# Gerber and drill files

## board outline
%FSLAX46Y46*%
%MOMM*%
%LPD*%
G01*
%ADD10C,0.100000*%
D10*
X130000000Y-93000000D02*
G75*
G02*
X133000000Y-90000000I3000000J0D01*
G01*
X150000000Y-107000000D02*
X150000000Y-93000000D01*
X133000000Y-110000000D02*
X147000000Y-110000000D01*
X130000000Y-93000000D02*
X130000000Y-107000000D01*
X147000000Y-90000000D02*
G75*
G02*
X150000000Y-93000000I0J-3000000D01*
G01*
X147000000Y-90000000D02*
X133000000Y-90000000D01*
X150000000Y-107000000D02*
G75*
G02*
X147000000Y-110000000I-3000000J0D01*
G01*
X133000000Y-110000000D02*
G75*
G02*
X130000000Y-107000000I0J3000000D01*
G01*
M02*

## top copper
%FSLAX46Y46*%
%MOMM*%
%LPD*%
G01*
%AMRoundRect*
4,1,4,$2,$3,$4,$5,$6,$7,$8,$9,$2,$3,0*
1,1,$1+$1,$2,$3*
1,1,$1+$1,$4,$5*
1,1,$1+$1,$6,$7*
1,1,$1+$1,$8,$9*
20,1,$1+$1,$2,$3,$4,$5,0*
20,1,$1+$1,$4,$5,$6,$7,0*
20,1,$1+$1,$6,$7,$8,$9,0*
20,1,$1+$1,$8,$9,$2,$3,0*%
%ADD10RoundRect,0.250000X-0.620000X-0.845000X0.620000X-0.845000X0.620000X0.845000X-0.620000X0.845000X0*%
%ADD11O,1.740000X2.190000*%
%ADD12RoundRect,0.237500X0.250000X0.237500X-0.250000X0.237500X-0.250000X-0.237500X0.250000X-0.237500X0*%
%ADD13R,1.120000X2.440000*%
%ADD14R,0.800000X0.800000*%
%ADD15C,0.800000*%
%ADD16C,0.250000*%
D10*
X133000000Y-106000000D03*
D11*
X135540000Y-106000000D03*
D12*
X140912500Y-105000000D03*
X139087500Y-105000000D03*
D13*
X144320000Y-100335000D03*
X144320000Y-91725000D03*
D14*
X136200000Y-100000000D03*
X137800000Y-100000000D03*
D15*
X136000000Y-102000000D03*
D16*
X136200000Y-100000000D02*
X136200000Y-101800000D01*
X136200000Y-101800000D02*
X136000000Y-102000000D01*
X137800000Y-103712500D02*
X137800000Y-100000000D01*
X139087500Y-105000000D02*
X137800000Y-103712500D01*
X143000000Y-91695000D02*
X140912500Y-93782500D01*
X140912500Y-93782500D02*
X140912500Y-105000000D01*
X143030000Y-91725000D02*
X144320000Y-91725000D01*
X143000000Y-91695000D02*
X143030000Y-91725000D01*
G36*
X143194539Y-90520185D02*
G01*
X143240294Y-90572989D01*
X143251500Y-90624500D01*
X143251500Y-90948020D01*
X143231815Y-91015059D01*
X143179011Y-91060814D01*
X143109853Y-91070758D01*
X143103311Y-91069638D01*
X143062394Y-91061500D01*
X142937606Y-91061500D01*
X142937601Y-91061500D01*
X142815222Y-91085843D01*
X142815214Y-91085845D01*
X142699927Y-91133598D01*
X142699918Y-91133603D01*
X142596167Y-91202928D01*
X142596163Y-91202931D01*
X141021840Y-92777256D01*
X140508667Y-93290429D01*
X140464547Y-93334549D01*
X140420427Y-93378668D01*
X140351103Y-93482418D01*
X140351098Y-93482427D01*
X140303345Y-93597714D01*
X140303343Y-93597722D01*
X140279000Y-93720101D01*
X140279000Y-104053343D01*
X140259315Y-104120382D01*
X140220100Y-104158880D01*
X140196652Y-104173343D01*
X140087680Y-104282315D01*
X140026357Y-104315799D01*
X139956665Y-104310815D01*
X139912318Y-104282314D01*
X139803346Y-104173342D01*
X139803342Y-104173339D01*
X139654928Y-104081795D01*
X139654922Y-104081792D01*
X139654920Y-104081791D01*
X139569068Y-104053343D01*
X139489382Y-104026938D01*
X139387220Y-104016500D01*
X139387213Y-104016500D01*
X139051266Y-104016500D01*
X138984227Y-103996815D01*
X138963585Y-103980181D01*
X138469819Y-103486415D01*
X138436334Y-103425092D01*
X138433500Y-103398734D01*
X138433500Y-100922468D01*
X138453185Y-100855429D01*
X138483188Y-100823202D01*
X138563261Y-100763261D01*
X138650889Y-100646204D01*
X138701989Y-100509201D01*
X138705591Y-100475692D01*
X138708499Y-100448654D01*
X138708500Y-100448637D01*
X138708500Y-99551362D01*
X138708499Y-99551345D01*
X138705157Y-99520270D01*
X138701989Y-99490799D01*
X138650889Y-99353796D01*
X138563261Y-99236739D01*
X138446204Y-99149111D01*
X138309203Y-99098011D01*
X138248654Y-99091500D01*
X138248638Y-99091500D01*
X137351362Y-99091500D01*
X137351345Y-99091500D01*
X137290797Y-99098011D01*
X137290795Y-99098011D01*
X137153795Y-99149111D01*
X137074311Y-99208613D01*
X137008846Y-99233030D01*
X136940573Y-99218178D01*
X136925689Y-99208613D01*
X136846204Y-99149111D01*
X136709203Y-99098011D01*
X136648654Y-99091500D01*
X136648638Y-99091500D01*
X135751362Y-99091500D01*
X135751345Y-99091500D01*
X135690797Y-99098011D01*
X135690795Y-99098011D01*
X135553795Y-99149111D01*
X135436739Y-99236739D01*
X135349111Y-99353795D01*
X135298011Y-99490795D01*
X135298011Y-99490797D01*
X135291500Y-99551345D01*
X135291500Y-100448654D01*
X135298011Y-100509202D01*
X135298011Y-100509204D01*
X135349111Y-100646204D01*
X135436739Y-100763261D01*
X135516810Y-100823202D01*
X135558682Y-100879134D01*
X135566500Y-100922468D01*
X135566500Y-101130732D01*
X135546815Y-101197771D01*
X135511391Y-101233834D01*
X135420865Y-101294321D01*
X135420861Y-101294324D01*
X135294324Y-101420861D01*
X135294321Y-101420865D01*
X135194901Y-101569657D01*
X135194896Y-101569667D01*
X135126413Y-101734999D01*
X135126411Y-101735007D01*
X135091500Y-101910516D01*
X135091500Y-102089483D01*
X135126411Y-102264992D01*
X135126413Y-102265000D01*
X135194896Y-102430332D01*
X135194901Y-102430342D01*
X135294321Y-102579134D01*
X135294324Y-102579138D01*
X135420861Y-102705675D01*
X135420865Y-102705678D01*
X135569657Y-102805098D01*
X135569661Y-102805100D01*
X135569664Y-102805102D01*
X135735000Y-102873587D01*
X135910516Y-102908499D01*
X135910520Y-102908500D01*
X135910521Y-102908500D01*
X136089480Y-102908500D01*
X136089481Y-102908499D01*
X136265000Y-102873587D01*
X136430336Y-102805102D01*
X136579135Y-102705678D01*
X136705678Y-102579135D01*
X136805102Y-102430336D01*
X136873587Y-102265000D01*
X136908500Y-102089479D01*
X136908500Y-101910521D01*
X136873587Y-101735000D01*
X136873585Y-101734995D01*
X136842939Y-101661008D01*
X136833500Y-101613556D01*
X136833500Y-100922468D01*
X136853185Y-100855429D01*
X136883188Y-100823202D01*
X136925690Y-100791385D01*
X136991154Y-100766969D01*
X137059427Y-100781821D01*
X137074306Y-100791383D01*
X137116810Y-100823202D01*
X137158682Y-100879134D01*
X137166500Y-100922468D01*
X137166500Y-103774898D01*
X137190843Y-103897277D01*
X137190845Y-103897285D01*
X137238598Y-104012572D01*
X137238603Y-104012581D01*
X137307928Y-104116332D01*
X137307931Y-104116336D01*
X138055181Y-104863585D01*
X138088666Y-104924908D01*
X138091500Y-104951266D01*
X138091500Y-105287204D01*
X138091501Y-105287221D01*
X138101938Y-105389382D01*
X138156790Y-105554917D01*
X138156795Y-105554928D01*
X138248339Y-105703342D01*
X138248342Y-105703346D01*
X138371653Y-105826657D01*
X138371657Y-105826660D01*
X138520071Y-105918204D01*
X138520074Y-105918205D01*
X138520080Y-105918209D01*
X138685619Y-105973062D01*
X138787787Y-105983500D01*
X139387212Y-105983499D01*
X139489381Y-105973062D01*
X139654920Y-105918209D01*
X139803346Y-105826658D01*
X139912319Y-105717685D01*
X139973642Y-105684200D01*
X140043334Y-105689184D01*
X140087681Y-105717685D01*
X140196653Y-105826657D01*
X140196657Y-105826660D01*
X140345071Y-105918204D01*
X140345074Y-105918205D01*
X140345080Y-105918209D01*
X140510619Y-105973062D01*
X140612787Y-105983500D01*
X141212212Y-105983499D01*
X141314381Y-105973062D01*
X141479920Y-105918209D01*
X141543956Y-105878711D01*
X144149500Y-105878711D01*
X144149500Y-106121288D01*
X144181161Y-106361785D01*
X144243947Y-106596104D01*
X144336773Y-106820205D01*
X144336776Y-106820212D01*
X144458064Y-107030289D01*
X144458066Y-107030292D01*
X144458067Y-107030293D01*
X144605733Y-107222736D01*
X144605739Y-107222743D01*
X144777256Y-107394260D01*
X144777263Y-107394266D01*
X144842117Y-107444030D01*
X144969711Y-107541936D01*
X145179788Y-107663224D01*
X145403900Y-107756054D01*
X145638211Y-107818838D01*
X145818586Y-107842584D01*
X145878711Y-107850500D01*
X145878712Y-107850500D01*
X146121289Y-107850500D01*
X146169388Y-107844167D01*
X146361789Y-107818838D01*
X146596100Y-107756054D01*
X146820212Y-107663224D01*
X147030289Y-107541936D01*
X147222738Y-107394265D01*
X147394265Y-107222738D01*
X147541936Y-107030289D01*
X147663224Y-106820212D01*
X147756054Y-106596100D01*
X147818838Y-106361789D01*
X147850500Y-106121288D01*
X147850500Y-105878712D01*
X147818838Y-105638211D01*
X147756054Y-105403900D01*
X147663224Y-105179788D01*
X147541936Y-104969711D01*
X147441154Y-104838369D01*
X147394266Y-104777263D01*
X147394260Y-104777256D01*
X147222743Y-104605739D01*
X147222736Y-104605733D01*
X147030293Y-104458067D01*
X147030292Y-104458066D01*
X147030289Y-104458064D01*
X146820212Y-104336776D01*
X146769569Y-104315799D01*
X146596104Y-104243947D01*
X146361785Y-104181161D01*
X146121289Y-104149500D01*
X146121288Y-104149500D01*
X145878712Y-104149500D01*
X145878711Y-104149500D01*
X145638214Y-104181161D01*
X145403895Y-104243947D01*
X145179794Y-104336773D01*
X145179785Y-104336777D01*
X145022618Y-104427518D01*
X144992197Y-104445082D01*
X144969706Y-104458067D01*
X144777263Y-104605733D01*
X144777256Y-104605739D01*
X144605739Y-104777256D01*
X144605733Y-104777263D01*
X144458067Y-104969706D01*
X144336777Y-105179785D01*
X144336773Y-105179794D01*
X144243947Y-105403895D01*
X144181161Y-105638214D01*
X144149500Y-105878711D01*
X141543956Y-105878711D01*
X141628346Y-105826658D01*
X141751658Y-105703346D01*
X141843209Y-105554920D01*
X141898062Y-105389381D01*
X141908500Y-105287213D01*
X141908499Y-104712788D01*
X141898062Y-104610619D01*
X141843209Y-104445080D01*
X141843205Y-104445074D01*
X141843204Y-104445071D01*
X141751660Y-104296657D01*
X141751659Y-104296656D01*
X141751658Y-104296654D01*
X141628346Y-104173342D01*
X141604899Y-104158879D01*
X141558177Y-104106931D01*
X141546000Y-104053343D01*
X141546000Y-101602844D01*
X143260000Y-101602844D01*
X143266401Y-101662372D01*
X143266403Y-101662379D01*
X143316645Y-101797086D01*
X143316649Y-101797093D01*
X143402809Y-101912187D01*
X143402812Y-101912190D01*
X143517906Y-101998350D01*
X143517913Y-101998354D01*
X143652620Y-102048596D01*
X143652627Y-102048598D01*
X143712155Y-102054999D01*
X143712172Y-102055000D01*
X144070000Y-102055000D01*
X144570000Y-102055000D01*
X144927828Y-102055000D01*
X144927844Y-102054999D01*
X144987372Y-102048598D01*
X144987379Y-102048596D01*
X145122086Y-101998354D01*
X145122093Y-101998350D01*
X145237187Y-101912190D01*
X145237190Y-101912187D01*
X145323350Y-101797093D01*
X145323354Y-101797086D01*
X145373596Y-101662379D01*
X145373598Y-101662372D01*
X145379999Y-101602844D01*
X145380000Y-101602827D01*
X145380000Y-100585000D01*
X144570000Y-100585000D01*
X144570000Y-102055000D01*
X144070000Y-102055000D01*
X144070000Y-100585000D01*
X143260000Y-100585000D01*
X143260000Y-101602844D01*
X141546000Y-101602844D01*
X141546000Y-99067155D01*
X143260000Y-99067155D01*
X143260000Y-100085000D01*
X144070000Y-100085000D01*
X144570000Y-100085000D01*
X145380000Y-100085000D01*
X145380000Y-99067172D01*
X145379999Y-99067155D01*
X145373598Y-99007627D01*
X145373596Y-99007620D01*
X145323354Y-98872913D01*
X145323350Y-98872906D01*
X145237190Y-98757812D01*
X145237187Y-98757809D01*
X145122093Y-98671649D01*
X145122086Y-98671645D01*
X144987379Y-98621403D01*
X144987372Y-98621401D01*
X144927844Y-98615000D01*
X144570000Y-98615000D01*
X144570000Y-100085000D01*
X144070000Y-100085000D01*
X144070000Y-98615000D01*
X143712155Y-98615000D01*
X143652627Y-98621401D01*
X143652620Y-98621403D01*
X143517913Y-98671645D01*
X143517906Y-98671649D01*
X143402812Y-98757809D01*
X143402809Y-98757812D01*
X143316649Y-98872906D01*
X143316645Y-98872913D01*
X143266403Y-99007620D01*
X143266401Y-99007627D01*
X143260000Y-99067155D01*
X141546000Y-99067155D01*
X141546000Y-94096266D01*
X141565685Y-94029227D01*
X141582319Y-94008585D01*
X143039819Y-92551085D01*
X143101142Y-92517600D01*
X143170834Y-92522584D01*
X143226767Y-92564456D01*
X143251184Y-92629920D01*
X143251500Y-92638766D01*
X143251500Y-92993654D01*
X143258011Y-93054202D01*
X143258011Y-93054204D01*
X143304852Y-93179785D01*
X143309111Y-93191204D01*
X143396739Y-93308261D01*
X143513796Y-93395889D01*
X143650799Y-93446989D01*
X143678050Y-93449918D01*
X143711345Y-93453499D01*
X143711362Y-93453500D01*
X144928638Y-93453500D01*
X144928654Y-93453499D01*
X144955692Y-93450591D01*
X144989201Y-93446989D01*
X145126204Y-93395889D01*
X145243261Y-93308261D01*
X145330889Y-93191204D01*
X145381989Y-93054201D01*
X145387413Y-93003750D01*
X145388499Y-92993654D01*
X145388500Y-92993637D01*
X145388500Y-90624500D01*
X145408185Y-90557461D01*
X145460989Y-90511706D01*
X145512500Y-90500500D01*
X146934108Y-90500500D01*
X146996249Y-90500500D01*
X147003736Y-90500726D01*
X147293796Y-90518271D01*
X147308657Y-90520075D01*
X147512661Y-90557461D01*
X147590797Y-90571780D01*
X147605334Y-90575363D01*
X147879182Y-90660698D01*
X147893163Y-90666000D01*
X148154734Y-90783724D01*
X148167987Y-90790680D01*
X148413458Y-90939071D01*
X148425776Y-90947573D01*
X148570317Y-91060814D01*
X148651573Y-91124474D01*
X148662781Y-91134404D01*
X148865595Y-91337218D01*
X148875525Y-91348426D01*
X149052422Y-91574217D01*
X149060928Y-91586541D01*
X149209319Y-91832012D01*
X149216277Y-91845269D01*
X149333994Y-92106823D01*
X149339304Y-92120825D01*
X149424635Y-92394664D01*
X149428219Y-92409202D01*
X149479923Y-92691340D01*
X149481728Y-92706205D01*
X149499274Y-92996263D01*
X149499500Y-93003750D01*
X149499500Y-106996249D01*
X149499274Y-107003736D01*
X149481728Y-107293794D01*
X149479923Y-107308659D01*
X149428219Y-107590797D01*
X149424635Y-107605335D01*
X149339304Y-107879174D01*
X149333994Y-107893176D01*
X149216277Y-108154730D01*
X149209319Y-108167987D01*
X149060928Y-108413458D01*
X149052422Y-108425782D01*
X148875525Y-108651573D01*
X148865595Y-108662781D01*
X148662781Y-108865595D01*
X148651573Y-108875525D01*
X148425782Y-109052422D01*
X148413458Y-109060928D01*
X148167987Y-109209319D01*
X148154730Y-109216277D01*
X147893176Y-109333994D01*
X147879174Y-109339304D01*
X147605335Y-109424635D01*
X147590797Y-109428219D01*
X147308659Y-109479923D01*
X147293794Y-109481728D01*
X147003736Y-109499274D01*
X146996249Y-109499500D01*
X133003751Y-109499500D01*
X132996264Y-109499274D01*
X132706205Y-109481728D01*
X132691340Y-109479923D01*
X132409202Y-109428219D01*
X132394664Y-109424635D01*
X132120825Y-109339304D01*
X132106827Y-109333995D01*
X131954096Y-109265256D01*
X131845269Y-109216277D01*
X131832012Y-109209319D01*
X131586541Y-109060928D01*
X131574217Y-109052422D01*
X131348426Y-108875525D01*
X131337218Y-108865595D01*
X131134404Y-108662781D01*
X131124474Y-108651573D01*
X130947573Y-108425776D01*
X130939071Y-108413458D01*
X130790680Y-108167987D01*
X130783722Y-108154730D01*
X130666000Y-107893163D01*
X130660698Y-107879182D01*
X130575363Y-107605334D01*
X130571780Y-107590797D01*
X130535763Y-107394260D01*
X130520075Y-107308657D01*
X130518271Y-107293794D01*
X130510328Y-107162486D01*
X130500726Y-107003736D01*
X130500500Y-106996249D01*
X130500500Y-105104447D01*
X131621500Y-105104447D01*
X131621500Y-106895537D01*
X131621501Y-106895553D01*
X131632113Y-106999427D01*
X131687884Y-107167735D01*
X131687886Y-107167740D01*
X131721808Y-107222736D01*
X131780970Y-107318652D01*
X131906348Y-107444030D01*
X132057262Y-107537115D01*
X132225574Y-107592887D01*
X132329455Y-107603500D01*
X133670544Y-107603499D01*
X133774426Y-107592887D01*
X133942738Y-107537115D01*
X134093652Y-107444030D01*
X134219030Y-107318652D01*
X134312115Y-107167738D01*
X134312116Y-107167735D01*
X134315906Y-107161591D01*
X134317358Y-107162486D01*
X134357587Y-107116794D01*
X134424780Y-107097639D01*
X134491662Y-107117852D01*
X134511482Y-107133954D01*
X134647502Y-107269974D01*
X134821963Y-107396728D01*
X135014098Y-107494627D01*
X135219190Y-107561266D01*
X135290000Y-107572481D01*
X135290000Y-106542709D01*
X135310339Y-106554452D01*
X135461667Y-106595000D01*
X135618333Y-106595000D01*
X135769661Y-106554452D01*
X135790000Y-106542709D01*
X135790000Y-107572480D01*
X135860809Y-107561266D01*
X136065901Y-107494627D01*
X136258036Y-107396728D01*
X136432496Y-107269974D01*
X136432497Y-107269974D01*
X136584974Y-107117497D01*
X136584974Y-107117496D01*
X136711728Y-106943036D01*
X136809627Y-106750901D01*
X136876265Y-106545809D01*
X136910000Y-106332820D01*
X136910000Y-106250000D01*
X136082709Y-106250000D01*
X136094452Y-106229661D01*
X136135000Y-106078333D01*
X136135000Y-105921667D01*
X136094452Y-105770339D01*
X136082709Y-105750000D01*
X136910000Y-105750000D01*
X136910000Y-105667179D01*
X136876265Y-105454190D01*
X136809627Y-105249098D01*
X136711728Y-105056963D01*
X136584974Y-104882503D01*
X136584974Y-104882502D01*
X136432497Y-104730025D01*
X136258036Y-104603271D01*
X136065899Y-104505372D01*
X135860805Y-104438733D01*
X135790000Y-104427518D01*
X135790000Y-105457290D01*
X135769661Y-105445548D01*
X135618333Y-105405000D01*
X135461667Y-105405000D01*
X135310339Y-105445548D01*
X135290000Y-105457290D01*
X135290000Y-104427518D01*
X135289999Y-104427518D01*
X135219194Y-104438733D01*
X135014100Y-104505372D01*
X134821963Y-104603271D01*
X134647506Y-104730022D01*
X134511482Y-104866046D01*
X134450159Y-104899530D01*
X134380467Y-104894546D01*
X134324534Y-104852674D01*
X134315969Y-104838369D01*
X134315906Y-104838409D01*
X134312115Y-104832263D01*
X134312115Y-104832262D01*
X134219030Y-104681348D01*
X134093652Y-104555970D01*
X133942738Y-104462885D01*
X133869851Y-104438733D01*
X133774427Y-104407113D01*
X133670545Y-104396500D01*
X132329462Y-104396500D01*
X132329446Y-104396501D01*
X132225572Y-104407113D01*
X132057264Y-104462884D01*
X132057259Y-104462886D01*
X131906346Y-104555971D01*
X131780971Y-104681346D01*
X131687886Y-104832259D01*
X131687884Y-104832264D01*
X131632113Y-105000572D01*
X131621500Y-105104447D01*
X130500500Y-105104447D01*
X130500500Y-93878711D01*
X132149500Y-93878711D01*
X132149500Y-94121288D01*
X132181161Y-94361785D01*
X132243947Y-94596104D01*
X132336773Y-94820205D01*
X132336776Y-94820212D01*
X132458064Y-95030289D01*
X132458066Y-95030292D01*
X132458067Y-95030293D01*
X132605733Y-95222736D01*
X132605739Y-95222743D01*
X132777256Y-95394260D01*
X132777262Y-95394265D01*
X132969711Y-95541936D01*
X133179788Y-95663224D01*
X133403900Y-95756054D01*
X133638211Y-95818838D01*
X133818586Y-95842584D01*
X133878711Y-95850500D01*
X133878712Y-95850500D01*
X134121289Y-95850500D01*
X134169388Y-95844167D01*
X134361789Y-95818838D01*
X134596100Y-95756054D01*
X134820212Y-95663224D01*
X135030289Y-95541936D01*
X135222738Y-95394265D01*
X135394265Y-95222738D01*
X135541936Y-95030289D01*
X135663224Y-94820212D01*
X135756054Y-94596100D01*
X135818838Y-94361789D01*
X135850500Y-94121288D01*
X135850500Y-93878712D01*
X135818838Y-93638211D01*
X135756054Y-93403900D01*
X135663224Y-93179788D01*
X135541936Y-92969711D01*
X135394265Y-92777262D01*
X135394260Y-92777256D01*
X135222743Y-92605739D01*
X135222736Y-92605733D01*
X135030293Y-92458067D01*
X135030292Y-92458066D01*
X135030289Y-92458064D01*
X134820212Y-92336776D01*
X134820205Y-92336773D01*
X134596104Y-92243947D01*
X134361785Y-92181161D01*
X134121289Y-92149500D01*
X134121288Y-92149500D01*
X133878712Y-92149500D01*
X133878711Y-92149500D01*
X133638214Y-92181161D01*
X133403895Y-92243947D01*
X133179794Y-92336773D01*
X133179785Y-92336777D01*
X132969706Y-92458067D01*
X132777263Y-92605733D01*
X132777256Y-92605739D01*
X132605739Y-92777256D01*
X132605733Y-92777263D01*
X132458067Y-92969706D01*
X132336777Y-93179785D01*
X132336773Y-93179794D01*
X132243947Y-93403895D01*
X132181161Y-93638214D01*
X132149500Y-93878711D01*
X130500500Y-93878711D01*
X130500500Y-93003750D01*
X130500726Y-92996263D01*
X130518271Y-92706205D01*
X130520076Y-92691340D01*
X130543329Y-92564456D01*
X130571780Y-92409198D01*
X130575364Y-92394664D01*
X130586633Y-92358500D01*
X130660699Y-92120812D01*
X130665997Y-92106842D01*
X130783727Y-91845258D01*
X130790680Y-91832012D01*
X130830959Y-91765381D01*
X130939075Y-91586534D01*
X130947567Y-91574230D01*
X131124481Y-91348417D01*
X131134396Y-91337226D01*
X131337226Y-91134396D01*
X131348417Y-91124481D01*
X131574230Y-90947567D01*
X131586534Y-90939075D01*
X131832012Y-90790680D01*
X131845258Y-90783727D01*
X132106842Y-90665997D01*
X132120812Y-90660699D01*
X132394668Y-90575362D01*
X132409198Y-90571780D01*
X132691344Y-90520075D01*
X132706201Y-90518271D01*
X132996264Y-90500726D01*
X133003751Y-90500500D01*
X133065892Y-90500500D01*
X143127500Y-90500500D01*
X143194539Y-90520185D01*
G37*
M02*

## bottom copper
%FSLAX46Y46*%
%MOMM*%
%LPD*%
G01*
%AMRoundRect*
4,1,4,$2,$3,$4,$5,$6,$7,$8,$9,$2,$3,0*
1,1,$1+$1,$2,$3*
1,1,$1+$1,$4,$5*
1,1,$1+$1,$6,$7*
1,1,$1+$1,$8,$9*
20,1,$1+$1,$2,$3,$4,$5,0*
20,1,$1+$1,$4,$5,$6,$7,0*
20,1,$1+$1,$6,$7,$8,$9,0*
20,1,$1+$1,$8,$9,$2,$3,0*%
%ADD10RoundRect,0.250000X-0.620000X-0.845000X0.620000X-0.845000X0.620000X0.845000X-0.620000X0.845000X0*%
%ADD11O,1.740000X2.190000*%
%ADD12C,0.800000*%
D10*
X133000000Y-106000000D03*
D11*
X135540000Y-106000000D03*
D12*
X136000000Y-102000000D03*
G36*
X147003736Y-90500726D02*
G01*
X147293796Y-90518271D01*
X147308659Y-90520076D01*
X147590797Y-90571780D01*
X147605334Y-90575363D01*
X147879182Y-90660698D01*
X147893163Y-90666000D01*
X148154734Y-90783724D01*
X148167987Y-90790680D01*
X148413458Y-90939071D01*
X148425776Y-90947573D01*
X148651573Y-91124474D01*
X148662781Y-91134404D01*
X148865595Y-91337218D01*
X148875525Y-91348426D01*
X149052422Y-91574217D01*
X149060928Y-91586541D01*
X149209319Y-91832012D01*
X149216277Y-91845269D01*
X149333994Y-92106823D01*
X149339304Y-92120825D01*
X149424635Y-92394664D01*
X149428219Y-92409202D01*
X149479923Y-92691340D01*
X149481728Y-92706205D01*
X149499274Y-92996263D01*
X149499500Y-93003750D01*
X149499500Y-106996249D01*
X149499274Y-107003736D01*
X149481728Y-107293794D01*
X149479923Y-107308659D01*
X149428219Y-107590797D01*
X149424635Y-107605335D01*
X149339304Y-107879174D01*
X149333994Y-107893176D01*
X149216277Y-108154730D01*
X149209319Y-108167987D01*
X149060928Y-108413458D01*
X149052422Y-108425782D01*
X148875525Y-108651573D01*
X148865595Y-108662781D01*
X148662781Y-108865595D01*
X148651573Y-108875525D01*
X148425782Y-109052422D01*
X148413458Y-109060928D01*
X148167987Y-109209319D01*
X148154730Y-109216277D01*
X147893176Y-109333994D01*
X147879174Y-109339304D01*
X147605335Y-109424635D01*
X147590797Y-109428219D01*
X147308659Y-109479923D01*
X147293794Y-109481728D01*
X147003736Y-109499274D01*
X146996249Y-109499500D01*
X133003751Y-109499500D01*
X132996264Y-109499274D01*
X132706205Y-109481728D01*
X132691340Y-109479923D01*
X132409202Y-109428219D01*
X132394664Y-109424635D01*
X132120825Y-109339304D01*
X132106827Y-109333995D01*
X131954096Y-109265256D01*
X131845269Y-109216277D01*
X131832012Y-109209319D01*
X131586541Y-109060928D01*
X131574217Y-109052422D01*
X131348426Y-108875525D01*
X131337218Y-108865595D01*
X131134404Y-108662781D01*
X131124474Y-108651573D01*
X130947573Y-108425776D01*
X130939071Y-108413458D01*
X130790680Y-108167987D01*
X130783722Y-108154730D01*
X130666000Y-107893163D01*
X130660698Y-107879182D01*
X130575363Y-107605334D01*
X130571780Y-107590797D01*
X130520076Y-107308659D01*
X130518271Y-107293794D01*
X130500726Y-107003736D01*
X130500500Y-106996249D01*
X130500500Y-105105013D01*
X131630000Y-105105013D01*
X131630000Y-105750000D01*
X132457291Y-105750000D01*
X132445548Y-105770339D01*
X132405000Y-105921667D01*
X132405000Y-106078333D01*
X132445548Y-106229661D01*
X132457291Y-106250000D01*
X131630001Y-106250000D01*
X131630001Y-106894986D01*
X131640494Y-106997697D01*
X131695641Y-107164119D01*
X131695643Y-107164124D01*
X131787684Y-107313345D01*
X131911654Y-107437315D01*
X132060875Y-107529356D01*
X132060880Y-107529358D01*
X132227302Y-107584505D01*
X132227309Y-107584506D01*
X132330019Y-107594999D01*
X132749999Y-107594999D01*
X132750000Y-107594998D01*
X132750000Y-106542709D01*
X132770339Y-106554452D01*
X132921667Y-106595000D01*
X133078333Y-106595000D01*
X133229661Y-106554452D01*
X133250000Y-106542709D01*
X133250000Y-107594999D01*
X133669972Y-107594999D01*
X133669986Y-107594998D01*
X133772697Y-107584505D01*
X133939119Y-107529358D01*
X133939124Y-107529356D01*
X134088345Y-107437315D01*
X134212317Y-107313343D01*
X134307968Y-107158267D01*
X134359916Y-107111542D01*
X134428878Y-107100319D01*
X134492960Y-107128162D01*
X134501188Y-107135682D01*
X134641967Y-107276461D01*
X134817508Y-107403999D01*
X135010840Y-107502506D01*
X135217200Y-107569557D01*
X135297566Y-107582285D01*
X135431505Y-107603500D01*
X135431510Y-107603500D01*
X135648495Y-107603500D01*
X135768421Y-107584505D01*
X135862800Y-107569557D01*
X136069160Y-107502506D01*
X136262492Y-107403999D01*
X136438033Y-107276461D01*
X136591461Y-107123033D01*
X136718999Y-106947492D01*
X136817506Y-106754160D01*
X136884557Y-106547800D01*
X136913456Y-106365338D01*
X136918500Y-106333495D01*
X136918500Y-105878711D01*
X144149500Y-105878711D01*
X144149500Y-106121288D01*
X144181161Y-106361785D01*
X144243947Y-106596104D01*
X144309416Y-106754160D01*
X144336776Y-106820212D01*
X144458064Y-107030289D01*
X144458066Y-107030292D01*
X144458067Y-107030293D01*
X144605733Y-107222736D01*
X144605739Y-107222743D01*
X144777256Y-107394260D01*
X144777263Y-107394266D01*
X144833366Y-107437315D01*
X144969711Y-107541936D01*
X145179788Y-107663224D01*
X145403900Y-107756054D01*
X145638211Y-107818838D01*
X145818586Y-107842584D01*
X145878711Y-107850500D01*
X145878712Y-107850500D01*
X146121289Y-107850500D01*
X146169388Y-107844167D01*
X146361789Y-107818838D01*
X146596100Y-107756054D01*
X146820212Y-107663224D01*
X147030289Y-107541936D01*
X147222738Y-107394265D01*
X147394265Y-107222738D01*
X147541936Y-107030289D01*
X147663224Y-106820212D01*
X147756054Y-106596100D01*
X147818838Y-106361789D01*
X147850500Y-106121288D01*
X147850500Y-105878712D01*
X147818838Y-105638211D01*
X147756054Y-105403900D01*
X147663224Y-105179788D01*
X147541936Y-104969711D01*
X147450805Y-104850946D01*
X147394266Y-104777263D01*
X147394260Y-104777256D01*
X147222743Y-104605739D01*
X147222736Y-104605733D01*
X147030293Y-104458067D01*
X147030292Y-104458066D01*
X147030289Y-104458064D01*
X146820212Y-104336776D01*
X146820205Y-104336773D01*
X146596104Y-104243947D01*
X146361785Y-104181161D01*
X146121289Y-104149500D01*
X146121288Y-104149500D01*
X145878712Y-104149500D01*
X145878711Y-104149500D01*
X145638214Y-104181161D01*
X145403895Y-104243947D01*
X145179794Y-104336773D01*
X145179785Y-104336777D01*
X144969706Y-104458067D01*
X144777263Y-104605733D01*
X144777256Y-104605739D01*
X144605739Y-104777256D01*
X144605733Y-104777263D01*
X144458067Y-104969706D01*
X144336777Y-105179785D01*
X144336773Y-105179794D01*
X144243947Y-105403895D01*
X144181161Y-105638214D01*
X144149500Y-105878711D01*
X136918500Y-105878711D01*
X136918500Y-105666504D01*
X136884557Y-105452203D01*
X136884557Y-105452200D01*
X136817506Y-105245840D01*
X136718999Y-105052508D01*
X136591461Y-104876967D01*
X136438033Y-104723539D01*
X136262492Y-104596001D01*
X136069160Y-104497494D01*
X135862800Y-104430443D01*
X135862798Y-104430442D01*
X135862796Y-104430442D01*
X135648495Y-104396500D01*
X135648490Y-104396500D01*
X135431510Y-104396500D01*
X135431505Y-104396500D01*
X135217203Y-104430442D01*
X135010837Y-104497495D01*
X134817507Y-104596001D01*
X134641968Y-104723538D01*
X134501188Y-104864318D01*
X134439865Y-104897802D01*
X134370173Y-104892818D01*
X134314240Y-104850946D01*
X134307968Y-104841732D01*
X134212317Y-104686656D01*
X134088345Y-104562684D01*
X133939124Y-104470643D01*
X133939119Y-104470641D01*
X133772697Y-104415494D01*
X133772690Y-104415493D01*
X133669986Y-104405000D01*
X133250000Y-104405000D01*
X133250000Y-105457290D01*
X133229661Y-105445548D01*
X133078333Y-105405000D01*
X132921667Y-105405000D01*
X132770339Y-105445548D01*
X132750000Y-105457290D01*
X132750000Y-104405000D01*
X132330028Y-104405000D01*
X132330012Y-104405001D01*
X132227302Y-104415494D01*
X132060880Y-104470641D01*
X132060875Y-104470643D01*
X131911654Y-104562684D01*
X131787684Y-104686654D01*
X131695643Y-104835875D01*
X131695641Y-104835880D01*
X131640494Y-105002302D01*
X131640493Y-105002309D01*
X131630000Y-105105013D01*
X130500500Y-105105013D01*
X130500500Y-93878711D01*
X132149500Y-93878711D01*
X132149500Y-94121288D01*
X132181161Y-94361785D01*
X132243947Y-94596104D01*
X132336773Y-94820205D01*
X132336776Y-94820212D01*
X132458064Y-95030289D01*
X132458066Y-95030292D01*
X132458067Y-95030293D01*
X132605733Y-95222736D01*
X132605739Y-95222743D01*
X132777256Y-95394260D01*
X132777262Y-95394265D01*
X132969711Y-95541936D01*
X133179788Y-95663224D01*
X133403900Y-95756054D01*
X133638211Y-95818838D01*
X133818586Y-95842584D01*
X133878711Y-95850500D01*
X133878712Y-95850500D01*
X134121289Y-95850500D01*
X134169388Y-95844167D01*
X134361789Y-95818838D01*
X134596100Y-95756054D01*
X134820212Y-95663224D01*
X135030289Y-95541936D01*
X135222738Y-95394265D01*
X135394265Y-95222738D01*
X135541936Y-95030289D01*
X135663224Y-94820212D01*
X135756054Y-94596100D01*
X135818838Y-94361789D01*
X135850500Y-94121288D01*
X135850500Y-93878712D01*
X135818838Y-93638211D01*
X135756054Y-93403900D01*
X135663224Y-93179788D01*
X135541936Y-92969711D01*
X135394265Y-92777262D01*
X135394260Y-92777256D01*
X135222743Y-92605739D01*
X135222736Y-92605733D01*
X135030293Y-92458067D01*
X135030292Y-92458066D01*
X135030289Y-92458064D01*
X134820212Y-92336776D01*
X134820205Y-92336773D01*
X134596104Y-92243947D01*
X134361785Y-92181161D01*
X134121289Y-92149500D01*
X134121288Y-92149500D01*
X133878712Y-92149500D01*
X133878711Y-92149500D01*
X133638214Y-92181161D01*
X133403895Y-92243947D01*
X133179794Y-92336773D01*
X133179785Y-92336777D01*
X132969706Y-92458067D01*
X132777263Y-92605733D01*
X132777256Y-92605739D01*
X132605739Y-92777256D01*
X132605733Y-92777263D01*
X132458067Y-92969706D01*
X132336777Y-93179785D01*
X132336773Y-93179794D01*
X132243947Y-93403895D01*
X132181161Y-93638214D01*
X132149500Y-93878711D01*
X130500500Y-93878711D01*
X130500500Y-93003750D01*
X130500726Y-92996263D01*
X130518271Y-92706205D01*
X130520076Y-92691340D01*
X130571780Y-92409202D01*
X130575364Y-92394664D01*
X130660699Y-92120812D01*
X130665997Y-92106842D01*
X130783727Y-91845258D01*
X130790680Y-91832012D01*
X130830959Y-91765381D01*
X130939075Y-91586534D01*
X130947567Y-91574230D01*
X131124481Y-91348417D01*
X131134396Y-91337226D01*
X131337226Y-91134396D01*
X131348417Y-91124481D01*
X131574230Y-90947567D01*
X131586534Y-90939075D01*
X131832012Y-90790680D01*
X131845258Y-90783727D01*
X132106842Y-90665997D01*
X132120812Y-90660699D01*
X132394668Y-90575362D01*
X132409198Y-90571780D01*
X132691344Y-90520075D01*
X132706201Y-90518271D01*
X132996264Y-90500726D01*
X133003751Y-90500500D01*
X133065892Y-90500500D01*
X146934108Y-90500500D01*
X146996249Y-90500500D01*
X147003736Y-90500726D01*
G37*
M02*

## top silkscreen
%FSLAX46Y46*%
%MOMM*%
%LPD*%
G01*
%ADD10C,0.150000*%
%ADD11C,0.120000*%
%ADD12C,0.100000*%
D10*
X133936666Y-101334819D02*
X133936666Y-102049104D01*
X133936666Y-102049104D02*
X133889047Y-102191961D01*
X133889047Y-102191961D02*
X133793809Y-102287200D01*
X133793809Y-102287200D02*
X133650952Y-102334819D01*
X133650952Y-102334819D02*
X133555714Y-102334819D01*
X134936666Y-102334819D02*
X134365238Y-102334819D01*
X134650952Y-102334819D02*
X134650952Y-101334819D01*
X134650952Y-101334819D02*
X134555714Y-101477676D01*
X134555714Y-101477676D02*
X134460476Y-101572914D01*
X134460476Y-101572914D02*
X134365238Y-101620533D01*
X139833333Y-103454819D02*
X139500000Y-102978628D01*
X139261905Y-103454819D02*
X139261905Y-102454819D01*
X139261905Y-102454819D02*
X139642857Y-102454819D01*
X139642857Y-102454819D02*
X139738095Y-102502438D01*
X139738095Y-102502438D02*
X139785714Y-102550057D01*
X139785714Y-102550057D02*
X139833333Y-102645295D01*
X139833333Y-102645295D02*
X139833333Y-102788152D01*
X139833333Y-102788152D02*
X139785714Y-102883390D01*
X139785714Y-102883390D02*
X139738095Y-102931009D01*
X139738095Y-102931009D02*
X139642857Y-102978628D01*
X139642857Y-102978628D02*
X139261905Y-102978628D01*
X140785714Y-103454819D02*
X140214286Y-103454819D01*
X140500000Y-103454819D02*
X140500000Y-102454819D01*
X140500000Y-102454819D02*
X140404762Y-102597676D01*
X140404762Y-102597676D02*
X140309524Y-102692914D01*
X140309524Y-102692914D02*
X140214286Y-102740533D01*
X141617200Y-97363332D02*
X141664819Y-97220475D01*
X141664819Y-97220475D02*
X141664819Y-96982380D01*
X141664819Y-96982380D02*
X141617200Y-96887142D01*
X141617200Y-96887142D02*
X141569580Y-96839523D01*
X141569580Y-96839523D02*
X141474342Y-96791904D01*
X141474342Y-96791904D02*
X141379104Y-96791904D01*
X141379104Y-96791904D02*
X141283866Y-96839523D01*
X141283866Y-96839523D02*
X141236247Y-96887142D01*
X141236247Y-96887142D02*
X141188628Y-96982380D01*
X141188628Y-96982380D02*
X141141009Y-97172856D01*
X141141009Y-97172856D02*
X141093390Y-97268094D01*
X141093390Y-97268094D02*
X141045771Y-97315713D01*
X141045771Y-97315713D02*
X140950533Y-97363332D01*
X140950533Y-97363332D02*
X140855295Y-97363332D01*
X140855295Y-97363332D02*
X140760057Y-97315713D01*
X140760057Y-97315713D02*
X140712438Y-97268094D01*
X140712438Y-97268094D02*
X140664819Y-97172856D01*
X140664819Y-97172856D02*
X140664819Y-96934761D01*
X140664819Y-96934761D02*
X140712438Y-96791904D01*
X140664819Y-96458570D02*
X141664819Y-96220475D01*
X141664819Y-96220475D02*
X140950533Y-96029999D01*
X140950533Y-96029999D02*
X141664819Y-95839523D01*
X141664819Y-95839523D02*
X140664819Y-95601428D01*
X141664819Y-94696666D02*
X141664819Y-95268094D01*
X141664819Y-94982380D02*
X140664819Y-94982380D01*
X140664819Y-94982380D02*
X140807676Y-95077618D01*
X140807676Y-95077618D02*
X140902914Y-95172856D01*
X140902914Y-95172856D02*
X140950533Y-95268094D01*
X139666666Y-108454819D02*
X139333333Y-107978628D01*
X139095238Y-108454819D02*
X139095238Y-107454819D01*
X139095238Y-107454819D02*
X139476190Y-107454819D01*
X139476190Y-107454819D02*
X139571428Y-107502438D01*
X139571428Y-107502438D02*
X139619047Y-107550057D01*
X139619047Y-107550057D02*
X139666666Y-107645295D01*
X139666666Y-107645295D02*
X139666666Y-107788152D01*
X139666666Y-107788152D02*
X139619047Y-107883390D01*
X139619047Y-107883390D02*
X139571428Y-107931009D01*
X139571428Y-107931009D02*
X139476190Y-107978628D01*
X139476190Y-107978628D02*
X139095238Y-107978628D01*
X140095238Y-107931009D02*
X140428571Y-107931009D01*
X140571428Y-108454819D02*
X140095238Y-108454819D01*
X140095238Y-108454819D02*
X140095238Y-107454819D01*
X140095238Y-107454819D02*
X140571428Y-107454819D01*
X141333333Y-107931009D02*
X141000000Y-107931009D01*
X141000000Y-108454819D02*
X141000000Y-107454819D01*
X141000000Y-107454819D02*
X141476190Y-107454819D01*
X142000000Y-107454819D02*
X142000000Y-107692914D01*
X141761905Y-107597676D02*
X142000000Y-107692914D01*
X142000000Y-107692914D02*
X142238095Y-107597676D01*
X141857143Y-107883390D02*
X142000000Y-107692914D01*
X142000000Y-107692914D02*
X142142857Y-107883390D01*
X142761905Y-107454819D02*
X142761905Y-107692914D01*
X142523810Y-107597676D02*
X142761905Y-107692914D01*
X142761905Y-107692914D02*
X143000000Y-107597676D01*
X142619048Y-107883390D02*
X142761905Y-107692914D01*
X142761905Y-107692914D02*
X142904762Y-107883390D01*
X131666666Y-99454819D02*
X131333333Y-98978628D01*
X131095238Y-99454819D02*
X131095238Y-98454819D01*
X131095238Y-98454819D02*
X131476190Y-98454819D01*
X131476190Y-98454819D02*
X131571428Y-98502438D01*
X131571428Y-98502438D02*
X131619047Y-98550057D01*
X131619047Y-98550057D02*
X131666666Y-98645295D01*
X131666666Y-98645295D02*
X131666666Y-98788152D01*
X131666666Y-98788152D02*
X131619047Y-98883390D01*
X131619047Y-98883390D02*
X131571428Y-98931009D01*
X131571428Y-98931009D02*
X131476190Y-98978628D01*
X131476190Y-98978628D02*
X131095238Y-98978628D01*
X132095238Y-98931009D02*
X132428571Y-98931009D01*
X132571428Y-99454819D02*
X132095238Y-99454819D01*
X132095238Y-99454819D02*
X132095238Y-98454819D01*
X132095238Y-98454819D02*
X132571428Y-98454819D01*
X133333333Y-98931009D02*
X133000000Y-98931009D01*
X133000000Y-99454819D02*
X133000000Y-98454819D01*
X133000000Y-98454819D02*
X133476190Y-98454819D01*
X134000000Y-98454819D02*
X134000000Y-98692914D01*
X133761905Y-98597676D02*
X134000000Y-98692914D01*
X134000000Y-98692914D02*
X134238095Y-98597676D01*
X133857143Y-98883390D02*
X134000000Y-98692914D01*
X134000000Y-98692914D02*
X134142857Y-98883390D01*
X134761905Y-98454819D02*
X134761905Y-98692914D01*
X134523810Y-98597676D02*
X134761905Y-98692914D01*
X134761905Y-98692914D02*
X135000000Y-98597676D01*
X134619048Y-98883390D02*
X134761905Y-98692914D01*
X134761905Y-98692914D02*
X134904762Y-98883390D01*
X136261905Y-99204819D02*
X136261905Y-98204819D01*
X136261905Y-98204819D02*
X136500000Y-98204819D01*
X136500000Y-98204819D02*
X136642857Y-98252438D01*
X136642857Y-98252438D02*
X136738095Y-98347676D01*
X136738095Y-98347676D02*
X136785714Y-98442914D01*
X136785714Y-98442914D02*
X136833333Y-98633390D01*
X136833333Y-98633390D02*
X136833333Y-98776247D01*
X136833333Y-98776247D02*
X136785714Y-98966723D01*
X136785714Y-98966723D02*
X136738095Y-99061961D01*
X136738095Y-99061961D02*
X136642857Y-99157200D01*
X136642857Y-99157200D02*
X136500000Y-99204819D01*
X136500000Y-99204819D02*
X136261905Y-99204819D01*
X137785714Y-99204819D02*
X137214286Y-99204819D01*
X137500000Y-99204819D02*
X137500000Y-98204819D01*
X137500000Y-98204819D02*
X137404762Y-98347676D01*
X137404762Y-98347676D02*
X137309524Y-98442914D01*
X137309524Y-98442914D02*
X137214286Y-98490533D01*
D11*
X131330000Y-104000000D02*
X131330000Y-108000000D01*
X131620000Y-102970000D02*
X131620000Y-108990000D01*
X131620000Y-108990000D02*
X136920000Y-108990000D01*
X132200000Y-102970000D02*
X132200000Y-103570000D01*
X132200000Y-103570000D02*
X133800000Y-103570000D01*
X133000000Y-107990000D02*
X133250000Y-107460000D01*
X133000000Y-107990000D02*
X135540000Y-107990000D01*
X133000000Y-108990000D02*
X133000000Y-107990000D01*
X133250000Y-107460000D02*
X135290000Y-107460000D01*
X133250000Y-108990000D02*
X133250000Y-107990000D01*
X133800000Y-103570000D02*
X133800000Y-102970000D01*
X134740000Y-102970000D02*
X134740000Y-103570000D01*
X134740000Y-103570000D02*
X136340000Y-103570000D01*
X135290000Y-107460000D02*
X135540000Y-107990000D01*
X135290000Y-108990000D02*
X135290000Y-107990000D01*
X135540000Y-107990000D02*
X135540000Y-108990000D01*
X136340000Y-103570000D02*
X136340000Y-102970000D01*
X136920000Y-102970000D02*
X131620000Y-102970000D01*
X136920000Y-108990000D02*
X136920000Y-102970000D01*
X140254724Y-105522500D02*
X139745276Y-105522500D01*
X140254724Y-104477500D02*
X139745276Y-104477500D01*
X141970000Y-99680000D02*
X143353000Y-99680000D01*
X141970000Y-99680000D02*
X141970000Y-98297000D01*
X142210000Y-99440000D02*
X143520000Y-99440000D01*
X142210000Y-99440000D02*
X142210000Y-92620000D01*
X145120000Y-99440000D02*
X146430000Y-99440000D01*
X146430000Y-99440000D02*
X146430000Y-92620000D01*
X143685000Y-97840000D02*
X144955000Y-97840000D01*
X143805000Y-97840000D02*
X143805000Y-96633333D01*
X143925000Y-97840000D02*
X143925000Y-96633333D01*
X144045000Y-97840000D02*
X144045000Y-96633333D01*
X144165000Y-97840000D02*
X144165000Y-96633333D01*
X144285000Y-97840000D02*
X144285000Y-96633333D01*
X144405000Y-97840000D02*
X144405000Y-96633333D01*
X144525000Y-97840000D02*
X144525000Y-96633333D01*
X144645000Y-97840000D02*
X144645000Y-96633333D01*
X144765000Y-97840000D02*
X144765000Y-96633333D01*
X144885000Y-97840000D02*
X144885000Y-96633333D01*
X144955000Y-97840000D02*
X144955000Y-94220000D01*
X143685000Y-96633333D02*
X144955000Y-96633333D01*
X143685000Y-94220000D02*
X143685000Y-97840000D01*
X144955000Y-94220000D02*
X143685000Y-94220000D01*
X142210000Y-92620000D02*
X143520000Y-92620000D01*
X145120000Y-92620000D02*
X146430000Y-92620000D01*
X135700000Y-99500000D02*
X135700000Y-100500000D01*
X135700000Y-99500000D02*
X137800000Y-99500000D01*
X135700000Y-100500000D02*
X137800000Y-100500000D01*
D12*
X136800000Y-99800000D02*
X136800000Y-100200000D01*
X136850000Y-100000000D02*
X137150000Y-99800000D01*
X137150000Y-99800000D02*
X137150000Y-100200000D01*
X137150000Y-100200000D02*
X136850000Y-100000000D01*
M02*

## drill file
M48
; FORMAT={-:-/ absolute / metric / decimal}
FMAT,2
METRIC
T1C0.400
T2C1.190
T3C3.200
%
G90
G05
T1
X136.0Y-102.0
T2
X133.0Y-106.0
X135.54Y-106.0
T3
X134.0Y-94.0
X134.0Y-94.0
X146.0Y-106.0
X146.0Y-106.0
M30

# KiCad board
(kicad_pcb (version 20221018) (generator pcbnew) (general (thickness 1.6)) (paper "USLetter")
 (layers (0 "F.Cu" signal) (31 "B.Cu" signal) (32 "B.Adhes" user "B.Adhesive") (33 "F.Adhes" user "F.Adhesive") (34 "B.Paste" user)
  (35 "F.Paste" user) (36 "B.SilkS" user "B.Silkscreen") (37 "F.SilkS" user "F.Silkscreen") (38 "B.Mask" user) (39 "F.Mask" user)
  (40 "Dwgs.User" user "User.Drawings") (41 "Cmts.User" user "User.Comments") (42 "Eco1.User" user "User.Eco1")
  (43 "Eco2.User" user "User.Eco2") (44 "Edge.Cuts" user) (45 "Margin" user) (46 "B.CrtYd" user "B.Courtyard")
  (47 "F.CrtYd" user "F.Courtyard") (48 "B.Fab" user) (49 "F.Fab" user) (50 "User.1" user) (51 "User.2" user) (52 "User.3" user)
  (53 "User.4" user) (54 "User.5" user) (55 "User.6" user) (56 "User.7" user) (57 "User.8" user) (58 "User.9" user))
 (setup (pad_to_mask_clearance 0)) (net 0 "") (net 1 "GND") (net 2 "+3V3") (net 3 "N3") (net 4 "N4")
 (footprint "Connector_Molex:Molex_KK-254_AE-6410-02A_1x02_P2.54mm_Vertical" (layer "F.Cu") (at 133 106)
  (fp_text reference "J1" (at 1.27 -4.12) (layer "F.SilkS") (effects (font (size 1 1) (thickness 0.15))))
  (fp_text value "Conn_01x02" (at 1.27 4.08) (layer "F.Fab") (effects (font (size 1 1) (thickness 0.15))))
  (fp_line (start -1.67 -2) (end -1.67 2) (stroke (width 0.12) (type solid)) (layer "F.SilkS"))
  (fp_line (start -1.38 -3.03) (end -1.38 2.99) (stroke (width 0.12) (type solid)) (layer "F.SilkS"))
  (fp_line (start -1.38 2.99) (end 3.92 2.99) (stroke (width 0.12) (type solid)) (layer "F.SilkS"))
  (fp_line (start -0.8 -3.03) (end -0.8 -2.43) (stroke (width 0.12) (type solid)) (layer "F.SilkS"))
  (fp_line (start -0.8 -2.43) (end 0.8 -2.43) (stroke (width 0.12) (type solid)) (layer "F.SilkS"))
  (fp_line (start 0 1.99) (end 0.25 1.46) (stroke (width 0.12) (type solid)) (layer "F.SilkS"))
  (fp_line (start 0 1.99) (end 2.54 1.99) (stroke (width 0.12) (type solid)) (layer "F.SilkS"))
  (fp_line (start 0 2.99) (end 0 1.99) (stroke (width 0.12) (type solid)) (layer "F.SilkS"))
  (fp_line (start 0.25 1.46) (end 2.29 1.46) (stroke (width 0.12) (type solid)) (layer "F.SilkS"))
  (fp_line (start 0.25 2.99) (end 0.25 1.99) (stroke (width 0.12) (type solid)) (layer "F.SilkS"))
  (fp_line (start 0.8 -2.43) (end 0.8 -3.03) (stroke (width 0.12) (type solid)) (layer "F.SilkS"))
  (fp_line (start 1.74 -3.03) (end 1.74 -2.43) (stroke (width 0.12) (type solid)) (layer "F.SilkS"))
  (fp_line (start 1.74 -2.43) (end 3.34 -2.43) (stroke (width 0.12) (type solid)) (layer "F.SilkS"))
  (fp_line (start 2.29 1.46) (end 2.54 1.99) (stroke (width 0.12) (type solid)) (layer "F.SilkS"))
  (fp_line (start 2.29 2.99) (end 2.29 1.99) (stroke (width 0.12) (type solid)) (layer "F.SilkS"))
  (fp_line (start 2.54 1.99) (end 2.54 2.99) (stroke (width 0.12) (type solid)) (layer "F.SilkS"))
  (fp_line (start 3.34 -2.43) (end 3.34 -3.03) (stroke (width 0.12) (type solid)) (layer "F.SilkS"))
  (fp_line (start 3.92 -3.03) (end -1.38 -3.03) (stroke (width 0.12) (type solid)) (layer "F.SilkS"))
  (fp_line (start 3.92 2.99) (end 3.92 -3.03) (stroke (width 0.12) (type solid)) (layer "F.SilkS"))
  (pad "1" thru_hole roundrect (at 0 0) (size 1.74 2.19) (drill 1.19) (layers "*.Cu" "*.Mask") (roundrect_rratio 0.143678) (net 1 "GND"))
  (pad "2" thru_hole oval (at 2.54 0) (size 1.74 2.19) (drill 1.19) (layers "*.Cu" "*.Mask") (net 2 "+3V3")))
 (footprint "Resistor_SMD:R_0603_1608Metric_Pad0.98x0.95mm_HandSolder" (layer "F.Cu") (at 140 105 180)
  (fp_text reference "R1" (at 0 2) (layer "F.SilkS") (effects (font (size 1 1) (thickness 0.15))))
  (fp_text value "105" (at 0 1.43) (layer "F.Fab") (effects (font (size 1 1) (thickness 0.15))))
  (fp_line (start -0.254724 -0.5225) (end 0.254724 -0.5225) (stroke (width 0.12) (type solid)) (layer "F.SilkS"))
  (fp_line (start -0.254724 0.5225) (end 0.254724 0.5225) (stroke (width 0.12) (type solid)) (layer "F.SilkS"))
  (pad "1" smd roundrect (at -0.9125 0 180) (size 0.975 0.95) (layers "F.Cu" "F.Paste" "F.Mask") (roundrect_rratio 0.25) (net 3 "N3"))
  (pad "2" smd roundrect (at 0.9125 0 180) (size 0.975 0.95) (layers "F.Cu" "F.Paste" "F.Mask") (roundrect_rratio 0.25) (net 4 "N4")))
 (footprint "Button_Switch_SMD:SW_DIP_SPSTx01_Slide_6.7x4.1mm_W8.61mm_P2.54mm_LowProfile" (layer "F.Cu") (at 144.32 96.03 90)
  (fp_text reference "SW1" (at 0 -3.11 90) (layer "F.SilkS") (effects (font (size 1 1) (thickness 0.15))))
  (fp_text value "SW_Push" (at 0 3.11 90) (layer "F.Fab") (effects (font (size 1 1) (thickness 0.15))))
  (fp_line (start -3.65 -2.35) (end -3.65 -0.967) (stroke (width 0.12) (type solid)) (layer "F.SilkS"))
  (fp_line (start -3.65 -2.35) (end -2.267 -2.35) (stroke (width 0.12) (type solid)) (layer "F.SilkS"))
  (fp_line (start -3.41 -2.11) (end -3.41 -0.8) (stroke (width 0.12) (type solid)) (layer "F.SilkS"))
  (fp_line (start -3.41 -2.11) (end 3.41 -2.11) (stroke (width 0.12) (type solid)) (layer "F.SilkS"))
  (fp_line (start -3.41 0.8) (end -3.41 2.11) (stroke (width 0.12) (type solid)) (layer "F.SilkS"))
  (fp_line (start -3.41 2.11) (end 3.41 2.11) (stroke (width 0.12) (type solid)) (layer "F.SilkS"))
  (fp_line (start -1.81 -0.635) (end -1.81 0.635) (stroke (width 0.12) (type solid)) (layer "F.SilkS"))
  (fp_line (start -1.81 -0.515) (end -0.603333 -0.515) (stroke (width 0.12) (type solid)) (layer "F.SilkS"))
  (fp_line (start -1.81 -0.395) (end -0.603333 -0.395) (stroke (width 0.12) (type solid)) (layer "F.SilkS"))
  (fp_line (start -1.81 -0.275) (end -0.603333 -0.275) (stroke (width 0.12) (type solid)) (layer "F.SilkS"))
  (fp_line (start -1.81 -0.155) (end -0.603333 -0.155) (stroke (width 0.12) (type solid)) (layer "F.SilkS"))
  (fp_line (start -1.81 -0.035) (end -0.603333 -0.035) (stroke (width 0.12) (type solid)) (layer "F.SilkS"))
  (fp_line (start -1.81 0.085) (end -0.603333 0.085) (stroke (width 0.12) (type solid)) (layer "F.SilkS"))
  (fp_line (start -1.81 0.205) (end -0.603333 0.205) (stroke (width 0.12) (type solid)) (layer "F.SilkS"))
  (fp_line (start -1.81 0.325) (end -0.603333 0.325) (stroke (width 0.12) (type solid)) (layer "F.SilkS"))
  (fp_line (start -1.81 0.445) (end -0.603333 0.445) (stroke (width 0.12) (type solid)) (layer "F.SilkS"))
  (fp_line (start -1.81 0.565) (end -0.603333 0.565) (stroke (width 0.12) (type solid)) (layer "F.SilkS"))
  (fp_line (start -1.81 0.635) (end 1.81 0.635) (stroke (width 0.12) (type solid)) (layer "F.SilkS"))
  (fp_line (start -0.603333 -0.635) (end -0.603333 0.635) (stroke (width 0.12) (type solid)) (layer "F.SilkS"))
  (fp_line (start 1.81 -0.635) (end -1.81 -0.635) (stroke (width 0.12) (type solid)) (layer "F.SilkS"))
  (fp_line (start 1.81 0.635) (end 1.81 -0.635) (stroke (width 0.12) (type solid)) (layer "F.SilkS"))
  (fp_line (start 3.41 -2.11) (end 3.41 -0.8) (stroke (width 0.12) (type solid)) (layer "F.SilkS"))
  (fp_line (start 3.41 0.8) (end 3.41 2.11) (stroke (width 0.12) (type solid)) (layer "F.SilkS"))
  (pad "1" smd rect (at -4.305 0 90) (size 2.44 1.12) (layers "F.Cu" "F.Paste" "F.Mask") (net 2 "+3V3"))
  (pad "2" smd rect (at 4.305 0 90) (size 2.44 1.12) (layers "F.Cu" "F.Paste" "F.Mask") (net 3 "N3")))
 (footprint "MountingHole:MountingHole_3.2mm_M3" (layer "F.Cu") (at 146 106)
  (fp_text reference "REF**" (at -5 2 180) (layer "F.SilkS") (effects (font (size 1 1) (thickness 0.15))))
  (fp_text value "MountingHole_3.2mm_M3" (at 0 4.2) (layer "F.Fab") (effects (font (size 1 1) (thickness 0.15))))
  (pad "" np_thru_hole circle (at 0 0) (size 3.2 3.2) (drill 3.2) (layers "*.Cu" "*.Mask"))
  (pad "" np_thru_hole circle (at 0 0) (size 3.2 3.2) (drill 3.2) (layers "*.Cu" "*.Mask")))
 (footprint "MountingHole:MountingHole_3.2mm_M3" (layer "F.Cu") (at 134 94)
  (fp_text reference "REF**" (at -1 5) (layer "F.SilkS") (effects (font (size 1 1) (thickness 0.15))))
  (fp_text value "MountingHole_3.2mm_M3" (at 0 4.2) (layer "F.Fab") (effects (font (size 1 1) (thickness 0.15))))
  (pad "" np_thru_hole circle (at 0 0) (size 3.2 3.2) (drill 3.2) (layers "*.Cu" "*.Mask"))
  (pad "" np_thru_hole circle (at 0 0) (size 3.2 3.2) (drill 3.2) (layers "*.Cu" "*.Mask")))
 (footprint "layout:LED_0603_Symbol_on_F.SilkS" (layer "F.Cu") (at 137 100)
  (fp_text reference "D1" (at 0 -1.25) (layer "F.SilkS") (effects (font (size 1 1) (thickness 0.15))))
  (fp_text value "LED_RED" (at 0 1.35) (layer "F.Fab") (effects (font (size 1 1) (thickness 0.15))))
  (fp_line (start -1.3 -0.5) (end -1.3 0.5) (stroke (width 0.12) (type solid)) (layer "F.SilkS"))
  (fp_line (start -1.3 -0.5) (end 0.8 -0.5) (stroke (width 0.12) (type solid)) (layer "F.SilkS"))
  (fp_line (start -1.3 0.5) (end 0.8 0.5) (stroke (width 0.12) (type solid)) (layer "F.SilkS"))
  (fp_line (start -0.2 -0.2) (end -0.2 0.2) (stroke (width 0.1) (type solid)) (layer "F.SilkS"))
  (fp_line (start -0.15 0) (end 0.15 -0.2) (stroke (width 0.1) (type solid)) (layer "F.SilkS"))
  (fp_line (start 0.15 -0.2) (end 0.15 0.2) (stroke (width 0.1) (type solid)) (layer "F.SilkS"))
  (fp_line (start 0.15 0.2) (end -0.15 0) (stroke (width 0.1) (type solid)) (layer "F.SilkS"))
  (pad "1" smd rect (at -0.8 0 180) (size 0.8 0.8) (layers "F.Cu" "F.Paste" "F.Mask") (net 1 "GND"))
  (pad "2" smd rect (at 0.8 0 180) (size 0.8 0.8) (layers "F.Cu" "F.Paste" "F.Mask") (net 4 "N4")))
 (gr_arc (start 130 93) (mid 130.87868 90.87868) (end 133 90) (stroke (width 0.1) (type default)) (layer "Edge.Cuts"))
 (gr_line (start 150 107) (end 150 93) (stroke (width 0.1) (type default)) (layer "Edge.Cuts"))
 (gr_line (start 133 110) (end 147 110) (stroke (width 0.1) (type default)) (layer "Edge.Cuts"))
 (gr_line (start 130 93) (end 130 107) (stroke (width 0.1) (type default)) (layer "Edge.Cuts"))
 (gr_arc (start 147 90) (mid 149.12132 90.87868) (end 150 93) (stroke (width 0.1) (type default)) (layer "Edge.Cuts"))
 (gr_line (start 147 90) (end 133 90) (stroke (width 0.1) (type default)) (layer "Edge.Cuts"))
 (gr_arc (start 150 107) (mid 149.12132 109.12132) (end 147 110) (stroke (width 0.1) (type default)) (layer "Edge.Cuts"))
 (gr_arc (start 133 110) (mid 130.87868 109.12132) (end 130 107) (stroke (width 0.1) (type default)) (layer "Edge.Cuts"))
 (segment (start 136.2 100) (end 136.2 101.8) (width 0.25) (layer "F.Cu") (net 1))
 (segment (start 136.2 101.8) (end 136 102) (width 0.25) (layer "F.Cu") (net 1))
 (via (at 136 102) (size 0.8) (drill 0.4) (layers "F.Cu" "B.Cu") (free) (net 1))
 (segment (start 137.8 103.7125) (end 137.8 100) (width 0.25) (layer "F.Cu") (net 4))
 (segment (start 139.0875 105) (end 137.8 103.7125) (width 0.25) (layer "F.Cu") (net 4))
 (segment (start 143 91.695) (end 140.9125 93.7825) (width 0.25) (layer "F.Cu") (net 3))
 (segment (start 140.9125 93.7825) (end 140.9125 105) (width 0.25) (layer "F.Cu") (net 3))
 (segment (start 143.03 91.725) (end 144.32 91.725) (width 0.25) (layer "F.Cu") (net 3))
 (segment (start 143 91.695) (end 143.03 91.725) (width 0.25) (layer "F.Cu") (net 3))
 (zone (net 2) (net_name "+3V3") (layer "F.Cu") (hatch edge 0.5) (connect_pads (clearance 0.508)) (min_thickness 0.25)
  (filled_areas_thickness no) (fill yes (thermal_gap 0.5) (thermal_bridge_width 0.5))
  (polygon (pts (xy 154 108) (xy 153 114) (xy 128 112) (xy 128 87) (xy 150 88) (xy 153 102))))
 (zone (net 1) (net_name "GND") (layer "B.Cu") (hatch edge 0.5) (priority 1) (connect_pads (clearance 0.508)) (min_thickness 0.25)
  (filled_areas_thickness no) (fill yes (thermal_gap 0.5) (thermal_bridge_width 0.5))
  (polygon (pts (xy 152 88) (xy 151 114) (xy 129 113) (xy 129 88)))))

